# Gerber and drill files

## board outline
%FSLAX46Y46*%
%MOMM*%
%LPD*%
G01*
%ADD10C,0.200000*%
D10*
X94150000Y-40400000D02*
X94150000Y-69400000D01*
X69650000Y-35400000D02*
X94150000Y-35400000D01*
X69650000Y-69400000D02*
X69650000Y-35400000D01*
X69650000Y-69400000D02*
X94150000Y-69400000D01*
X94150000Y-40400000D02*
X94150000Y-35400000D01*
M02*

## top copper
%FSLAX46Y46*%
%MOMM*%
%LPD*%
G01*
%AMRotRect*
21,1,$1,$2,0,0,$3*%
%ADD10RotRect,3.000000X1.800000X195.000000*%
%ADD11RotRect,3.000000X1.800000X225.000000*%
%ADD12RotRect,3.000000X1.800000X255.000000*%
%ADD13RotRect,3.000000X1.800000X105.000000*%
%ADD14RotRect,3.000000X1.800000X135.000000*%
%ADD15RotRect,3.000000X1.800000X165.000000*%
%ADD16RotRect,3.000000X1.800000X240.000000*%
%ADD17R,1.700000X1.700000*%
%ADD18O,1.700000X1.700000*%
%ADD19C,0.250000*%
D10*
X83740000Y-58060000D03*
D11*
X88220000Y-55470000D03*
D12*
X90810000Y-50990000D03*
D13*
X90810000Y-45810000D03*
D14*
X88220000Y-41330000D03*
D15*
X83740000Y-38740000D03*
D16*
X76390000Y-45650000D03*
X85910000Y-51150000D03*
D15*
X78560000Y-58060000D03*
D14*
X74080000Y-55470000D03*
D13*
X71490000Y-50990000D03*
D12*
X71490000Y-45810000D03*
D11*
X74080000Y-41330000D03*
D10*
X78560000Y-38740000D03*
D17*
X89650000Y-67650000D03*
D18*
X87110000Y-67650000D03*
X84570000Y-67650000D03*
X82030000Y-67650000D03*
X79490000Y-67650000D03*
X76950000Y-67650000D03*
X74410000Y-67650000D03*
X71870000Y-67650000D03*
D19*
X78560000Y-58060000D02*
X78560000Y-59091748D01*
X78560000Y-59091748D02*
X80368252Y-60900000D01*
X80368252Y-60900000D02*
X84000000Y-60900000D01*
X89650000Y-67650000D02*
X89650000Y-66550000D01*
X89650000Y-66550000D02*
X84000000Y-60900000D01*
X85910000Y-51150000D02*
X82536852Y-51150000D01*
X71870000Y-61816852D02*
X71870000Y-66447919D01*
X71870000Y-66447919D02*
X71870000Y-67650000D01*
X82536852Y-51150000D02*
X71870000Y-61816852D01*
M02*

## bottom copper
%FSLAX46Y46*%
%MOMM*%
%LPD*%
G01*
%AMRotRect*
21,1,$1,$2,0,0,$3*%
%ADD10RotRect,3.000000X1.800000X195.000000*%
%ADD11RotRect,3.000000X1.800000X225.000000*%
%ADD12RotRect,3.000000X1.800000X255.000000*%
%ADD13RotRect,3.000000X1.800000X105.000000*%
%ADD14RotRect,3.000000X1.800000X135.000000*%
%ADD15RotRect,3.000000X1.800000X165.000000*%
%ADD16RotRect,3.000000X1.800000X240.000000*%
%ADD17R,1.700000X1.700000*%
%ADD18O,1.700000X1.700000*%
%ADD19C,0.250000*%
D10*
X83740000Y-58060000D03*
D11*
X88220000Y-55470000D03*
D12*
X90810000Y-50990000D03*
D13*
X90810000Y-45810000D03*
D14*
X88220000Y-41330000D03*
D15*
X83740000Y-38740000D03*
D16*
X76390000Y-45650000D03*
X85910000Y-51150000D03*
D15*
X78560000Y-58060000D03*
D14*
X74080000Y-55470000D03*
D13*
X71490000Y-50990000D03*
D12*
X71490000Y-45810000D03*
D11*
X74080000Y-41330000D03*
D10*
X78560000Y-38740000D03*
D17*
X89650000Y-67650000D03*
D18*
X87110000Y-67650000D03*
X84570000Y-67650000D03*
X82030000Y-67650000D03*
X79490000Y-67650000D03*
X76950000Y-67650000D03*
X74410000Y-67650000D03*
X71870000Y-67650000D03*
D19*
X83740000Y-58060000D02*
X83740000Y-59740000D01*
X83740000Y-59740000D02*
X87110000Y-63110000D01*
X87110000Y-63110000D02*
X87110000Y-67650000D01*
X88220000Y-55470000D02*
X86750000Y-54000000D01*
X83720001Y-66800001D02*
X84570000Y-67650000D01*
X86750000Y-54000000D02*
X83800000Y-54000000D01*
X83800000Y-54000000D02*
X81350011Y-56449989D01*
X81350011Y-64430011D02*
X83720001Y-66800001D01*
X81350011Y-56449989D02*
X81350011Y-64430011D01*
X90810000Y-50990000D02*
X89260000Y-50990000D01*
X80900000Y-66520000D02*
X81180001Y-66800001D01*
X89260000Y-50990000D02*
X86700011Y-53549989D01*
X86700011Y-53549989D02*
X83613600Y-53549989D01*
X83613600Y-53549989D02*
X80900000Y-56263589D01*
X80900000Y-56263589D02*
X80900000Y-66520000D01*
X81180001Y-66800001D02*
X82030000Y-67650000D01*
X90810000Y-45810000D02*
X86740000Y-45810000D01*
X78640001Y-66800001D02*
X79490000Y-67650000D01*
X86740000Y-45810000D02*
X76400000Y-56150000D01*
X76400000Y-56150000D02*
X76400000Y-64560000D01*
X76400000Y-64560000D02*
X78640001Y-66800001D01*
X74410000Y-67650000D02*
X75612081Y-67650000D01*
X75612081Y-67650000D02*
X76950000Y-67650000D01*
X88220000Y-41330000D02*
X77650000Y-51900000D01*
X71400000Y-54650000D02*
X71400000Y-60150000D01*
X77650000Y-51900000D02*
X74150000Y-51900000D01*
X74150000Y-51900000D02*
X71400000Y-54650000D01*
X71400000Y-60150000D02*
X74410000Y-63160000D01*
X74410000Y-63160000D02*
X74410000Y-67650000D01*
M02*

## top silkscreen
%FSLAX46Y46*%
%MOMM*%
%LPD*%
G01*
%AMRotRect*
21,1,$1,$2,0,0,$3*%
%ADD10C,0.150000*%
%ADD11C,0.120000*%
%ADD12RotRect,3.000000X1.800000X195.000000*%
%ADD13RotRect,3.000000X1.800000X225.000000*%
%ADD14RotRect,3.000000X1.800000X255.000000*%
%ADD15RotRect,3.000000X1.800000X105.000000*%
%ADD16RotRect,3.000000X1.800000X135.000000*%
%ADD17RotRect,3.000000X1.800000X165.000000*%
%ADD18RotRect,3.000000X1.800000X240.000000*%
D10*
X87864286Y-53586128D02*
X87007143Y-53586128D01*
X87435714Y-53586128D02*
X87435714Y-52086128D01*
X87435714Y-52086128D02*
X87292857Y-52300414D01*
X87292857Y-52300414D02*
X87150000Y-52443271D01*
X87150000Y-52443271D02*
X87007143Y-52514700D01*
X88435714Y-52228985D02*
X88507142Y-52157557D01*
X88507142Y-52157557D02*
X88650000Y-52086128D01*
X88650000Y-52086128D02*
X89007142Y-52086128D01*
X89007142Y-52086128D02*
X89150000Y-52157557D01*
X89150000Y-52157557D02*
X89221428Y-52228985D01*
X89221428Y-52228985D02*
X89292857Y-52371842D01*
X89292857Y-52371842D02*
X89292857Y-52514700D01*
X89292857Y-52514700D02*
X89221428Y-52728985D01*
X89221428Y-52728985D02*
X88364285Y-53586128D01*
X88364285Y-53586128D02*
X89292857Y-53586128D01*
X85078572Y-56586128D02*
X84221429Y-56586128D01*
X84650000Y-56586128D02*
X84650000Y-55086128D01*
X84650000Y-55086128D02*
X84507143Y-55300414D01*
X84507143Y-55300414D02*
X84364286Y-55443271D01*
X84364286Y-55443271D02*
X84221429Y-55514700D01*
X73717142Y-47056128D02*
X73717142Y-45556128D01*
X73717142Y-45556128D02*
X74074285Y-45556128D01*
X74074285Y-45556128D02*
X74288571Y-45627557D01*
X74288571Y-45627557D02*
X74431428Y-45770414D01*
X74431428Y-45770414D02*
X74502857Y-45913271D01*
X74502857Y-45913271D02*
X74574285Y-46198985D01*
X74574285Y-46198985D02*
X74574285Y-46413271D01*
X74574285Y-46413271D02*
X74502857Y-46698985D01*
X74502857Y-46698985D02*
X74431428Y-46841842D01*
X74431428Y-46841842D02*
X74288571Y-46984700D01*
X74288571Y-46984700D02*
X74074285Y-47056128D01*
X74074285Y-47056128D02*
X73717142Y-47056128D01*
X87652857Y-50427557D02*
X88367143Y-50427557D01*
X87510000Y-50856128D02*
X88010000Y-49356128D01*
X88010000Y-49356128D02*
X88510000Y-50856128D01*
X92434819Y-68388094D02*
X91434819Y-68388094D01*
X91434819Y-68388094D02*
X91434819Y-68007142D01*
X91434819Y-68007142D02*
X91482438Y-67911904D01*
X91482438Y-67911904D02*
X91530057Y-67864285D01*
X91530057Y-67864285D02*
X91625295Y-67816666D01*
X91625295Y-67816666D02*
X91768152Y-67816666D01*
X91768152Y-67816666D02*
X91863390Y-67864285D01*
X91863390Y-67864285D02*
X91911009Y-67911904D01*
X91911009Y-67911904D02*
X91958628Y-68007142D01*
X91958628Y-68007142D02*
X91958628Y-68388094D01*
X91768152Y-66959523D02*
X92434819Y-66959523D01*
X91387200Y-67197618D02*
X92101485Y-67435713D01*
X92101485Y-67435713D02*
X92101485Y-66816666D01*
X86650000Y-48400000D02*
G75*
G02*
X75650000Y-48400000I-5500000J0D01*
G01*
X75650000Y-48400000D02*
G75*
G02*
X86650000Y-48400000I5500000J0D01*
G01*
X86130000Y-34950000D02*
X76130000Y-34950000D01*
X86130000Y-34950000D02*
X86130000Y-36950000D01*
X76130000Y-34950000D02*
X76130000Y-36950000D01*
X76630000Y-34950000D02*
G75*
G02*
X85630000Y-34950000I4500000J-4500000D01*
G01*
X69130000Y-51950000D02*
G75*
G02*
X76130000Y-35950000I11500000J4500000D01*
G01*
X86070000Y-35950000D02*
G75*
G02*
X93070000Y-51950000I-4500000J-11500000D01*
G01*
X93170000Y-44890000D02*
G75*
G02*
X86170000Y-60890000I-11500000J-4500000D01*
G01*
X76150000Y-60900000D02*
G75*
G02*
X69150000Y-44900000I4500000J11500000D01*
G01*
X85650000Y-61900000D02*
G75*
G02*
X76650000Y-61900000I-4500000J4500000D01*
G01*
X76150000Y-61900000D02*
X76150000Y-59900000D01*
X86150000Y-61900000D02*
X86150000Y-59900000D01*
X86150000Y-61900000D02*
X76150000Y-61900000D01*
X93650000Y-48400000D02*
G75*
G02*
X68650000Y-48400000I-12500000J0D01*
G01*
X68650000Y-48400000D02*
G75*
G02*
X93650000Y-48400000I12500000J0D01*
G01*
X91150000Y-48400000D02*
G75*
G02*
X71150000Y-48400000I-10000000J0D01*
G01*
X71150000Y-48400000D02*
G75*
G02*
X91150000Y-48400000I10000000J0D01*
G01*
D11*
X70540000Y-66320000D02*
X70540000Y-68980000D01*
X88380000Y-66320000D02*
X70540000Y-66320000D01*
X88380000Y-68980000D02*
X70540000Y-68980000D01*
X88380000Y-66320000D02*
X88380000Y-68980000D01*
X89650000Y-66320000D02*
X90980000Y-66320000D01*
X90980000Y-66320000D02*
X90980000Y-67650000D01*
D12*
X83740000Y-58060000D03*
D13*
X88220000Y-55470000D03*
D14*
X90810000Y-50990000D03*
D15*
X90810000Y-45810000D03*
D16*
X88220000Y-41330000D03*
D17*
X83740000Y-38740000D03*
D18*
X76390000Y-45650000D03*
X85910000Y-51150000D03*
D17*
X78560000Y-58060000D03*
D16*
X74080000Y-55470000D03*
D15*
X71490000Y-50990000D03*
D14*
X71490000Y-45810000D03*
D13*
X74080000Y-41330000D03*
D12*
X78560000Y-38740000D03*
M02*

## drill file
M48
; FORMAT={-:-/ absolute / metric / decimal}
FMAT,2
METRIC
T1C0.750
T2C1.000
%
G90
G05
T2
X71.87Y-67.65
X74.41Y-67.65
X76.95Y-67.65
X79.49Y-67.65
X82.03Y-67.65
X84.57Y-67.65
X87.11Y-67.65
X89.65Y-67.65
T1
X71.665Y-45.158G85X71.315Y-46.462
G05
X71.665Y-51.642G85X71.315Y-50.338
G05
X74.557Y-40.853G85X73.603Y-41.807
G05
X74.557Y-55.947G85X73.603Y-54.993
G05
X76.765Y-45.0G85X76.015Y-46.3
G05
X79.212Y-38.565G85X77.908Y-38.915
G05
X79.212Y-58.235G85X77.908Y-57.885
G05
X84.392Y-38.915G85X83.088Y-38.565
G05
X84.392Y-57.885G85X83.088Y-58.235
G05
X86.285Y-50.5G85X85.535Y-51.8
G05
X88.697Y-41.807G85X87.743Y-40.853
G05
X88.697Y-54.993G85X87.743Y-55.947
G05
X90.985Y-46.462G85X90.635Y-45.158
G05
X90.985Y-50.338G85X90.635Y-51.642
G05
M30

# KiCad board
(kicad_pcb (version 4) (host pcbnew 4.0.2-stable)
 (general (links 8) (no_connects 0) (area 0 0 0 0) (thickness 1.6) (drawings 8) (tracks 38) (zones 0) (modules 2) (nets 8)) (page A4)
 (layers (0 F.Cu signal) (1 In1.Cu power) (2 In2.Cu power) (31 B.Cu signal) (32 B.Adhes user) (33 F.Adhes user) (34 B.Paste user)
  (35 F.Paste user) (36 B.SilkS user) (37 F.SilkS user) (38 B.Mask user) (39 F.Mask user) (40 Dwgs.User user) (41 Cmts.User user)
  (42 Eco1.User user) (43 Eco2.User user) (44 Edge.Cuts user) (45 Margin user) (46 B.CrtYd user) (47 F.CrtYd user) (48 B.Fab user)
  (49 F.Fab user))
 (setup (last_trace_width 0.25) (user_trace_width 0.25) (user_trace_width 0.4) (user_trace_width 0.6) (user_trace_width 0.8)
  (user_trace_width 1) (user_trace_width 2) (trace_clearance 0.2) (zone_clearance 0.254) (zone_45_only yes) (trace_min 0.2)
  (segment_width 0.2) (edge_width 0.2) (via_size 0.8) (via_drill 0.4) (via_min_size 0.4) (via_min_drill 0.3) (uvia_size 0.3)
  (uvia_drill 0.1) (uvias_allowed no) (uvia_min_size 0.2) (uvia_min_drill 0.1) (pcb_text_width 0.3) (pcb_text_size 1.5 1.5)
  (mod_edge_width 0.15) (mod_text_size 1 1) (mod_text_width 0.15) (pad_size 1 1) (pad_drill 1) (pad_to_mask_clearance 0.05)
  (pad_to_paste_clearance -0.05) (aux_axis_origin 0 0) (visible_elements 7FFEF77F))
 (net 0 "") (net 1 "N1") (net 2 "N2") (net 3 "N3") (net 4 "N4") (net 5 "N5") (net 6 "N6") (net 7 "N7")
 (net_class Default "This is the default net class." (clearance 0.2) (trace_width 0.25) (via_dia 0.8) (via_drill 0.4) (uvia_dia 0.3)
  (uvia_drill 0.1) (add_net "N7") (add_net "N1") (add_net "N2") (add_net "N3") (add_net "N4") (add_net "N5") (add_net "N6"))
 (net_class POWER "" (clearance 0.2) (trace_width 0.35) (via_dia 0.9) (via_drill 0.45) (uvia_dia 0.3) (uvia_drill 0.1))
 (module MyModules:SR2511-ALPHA (layer F.Cu) (at 81.15 48.4 180)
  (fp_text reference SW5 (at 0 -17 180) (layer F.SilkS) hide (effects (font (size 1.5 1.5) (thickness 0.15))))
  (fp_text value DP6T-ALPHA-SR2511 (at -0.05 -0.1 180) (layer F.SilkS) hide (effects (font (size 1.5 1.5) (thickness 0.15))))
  (fp_circle (center 0 0) (end 0 -5.5) (layer F.SilkS) (width 0.15))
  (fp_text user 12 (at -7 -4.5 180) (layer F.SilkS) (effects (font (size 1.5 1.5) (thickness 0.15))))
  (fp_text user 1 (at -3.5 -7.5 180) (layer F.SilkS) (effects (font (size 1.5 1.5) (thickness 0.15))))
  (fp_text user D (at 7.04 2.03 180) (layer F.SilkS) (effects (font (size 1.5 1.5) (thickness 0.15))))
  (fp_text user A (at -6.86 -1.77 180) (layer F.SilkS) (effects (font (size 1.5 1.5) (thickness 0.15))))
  (fp_line (start -4.98 13.45) (end 5.02 13.45) (layer F.SilkS) (width 0.15))
  (fp_line (start -4.98 13.45) (end -4.98 11.45) (layer F.SilkS) (width 0.15))
  (fp_line (start 5.02 13.45) (end 5.02 11.45) (layer F.SilkS) (width 0.15))
  (fp_arc (start 0.02 8.95) (end -4.48 13.45) (angle -90) (layer F.SilkS) (width 0.15))
  (fp_arc (start 0.52 0.95) (end 5.02 12.45) (angle -90) (layer F.SilkS) (width 0.15))
  (fp_arc (start -0.42 0.95) (end -4.92 12.45) (angle 90) (layer F.SilkS) (width 0.15))
  (fp_arc (start -0.52 -0.99) (end -5.02 -12.49) (angle -90) (layer F.SilkS) (width 0.15))
  (fp_arc (start 0.5 -1) (end 5 -12.5) (angle 90) (layer F.SilkS) (width 0.15))
  (fp_arc (start 0 -9) (end -4.5 -13.5) (angle 90) (layer F.SilkS) (width 0.15))
  (fp_line (start 5 -13.5) (end 5 -11.5) (layer F.SilkS) (width 0.15))
  (fp_line (start -5 -13.5) (end -5 -11.5) (layer F.SilkS) (width 0.15))
  (fp_line (start -5 -13.5) (end 5 -13.5) (layer F.SilkS) (width 0.15))
  (fp_circle (center 0 0) (end 12.5 0) (layer F.SilkS) (width 0.15))
  (fp_circle (center 0 0) (end 0 -10) (layer F.SilkS) (width 0.15))
  (pad 1 thru_hole rect (at -2.59 -9.66 195) (size 3 1.8) (drill oval 2.1 0.75) (layers *.Cu *.Mask F.SilkS) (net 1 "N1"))
  (pad 12 thru_hole rect (at -7.07 -7.07 225) (size 3 1.8) (drill oval 2.1 0.75) (layers *.Cu *.Mask F.SilkS) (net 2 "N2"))
  (pad 11 thru_hole rect (at -9.66 -2.59 255) (size 3 1.8) (drill oval 2.1 0.75) (layers *.Cu *.Mask F.SilkS) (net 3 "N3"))
  (pad 10 thru_hole rect (at -9.66 2.59 105) (size 3 1.8) (drill oval 2.1 0.75) (layers *.Cu *.Mask F.SilkS) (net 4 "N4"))
  (pad 9 thru_hole rect (at -7.07 7.07 135) (size 3 1.8) (drill oval 2.1 0.75) (layers *.Cu *.Mask F.SilkS) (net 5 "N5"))
  (pad 8 thru_hole rect (at -2.59 9.66 165) (size 3 1.8) (drill oval 2.1 0.75) (layers *.Cu *.Mask F.SilkS))
  (pad D thru_hole rect (at 4.76 2.75 240) (size 3 1.8) (drill oval 2.25 0.75) (layers *.Cu *.Mask F.SilkS))
  (pad A thru_hole rect (at -4.76 -2.75 240) (size 3 1.8) (drill oval 2.25 0.75) (layers *.Cu *.Mask F.SilkS) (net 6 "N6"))
  (pad 2 thru_hole rect (at 2.59 -9.66 165) (size 3 1.8) (drill oval 2.1 0.75) (layers *.Cu *.Mask F.SilkS) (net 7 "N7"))
  (pad 3 thru_hole rect (at 7.07 -7.07 135) (size 3 1.8) (drill oval 2.1 0.75) (layers *.Cu *.Mask F.SilkS))
  (pad 4 thru_hole rect (at 9.66 -2.59 105) (size 3 1.8) (drill oval 2.1 0.75) (layers *.Cu *.Mask F.SilkS))
  (pad 5 thru_hole rect (at 9.66 2.59 255) (size 3 1.8) (drill oval 2.1 0.75) (layers *.Cu *.Mask F.SilkS))
  (pad 6 thru_hole rect (at 7.07 7.07 225) (size 3 1.8) (drill oval 2.1 0.75) (layers *.Cu *.Mask F.SilkS))
  (pad 7 thru_hole rect (at 2.59 9.66 195) (size 3 1.8) (drill oval 2.1 0.75) (layers *.Cu *.Mask F.SilkS)))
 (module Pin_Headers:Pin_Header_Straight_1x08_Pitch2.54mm (layer F.Cu) (at 89.65 67.65 270)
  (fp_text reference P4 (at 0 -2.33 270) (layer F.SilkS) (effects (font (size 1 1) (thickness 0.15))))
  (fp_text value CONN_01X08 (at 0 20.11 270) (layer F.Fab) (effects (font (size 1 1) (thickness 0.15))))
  (fp_line (start -1.33 19.11) (end 1.33 19.11) (layer F.SilkS) (width 0.12))
  (fp_line (start -1.33 1.27) (end -1.33 19.11) (layer F.SilkS) (width 0.12))
  (fp_line (start 1.33 1.27) (end 1.33 19.11) (layer F.SilkS) (width 0.12))
  (fp_line (start -1.33 1.27) (end 1.33 1.27) (layer F.SilkS) (width 0.12))
  (fp_line (start -1.33 0) (end -1.33 -1.33) (layer F.SilkS) (width 0.12))
  (fp_line (start -1.33 -1.33) (end 0 -1.33) (layer F.SilkS) (width 0.12))
  (pad 1 thru_hole rect (at 0 0 270) (size 1.7 1.7) (drill 1) (layers *.Cu *.Mask) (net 7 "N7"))
  (pad 2 thru_hole oval (at 0 2.54 270) (size 1.7 1.7) (drill 1) (layers *.Cu *.Mask) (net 1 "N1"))
  (pad 3 thru_hole oval (at 0 5.08 270) (size 1.7 1.7) (drill 1) (layers *.Cu *.Mask) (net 2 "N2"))
  (pad 4 thru_hole oval (at 0 7.62 270) (size 1.7 1.7) (drill 1) (layers *.Cu *.Mask) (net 3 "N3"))
  (pad 5 thru_hole oval (at 0 10.16 270) (size 1.7 1.7) (drill 1) (layers *.Cu *.Mask) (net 4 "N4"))
  (pad 6 thru_hole oval (at 0 12.7 270) (size 1.7 1.7) (drill 1) (layers *.Cu *.Mask) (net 5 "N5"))
  (pad 7 thru_hole oval (at 0 15.24 270) (size 1.7 1.7) (drill 1) (layers *.Cu *.Mask) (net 5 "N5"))
  (pad 8 thru_hole oval (at 0 17.78 270) (size 1.7 1.7) (drill 1) (layers *.Cu *.Mask) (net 6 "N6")))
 (gr_line (start 94.15 40.4) (end 94.15 69.4) (layer Edge.Cuts) (width 0.2))
 (gr_line (start 69.65 35.4) (end 94.15 35.4) (layer Edge.Cuts) (width 0.2))
 (gr_line (start 69.65 69.4) (end 69.65 35.4) (layer Edge.Cuts) (width 0.2))
 (gr_line (start 69.65 69.4) (end 94.15 69.4) (layer Edge.Cuts) (width 0.2))
 (gr_line (start 94.15 40.4) (end 94.15 35.4) (layer Edge.Cuts) (width 0.2))
 (segment (start 78.56 58.06) (end 78.56 59.091748) (width 0.25) (layer F.Cu) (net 7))
 (segment (start 78.56 59.091748) (end 80.368252 60.9) (width 0.25) (layer F.Cu) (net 7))
 (segment (start 80.368252 60.9) (end 84 60.9) (width 0.25) (layer F.Cu) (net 7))
 (segment (start 89.65 67.65) (end 89.65 66.55) (width 0.25) (layer F.Cu) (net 7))
 (segment (start 89.65 66.55) (end 84 60.9) (width 0.25) (layer F.Cu) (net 7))
 (segment (start 83.74 58.06) (end 83.74 59.74) (width 0.25) (layer B.Cu) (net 1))
 (segment (start 83.74 59.74) (end 87.11 63.11) (width 0.25) (layer B.Cu) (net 1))
 (segment (start 87.11 63.11) (end 87.11 67.65) (width 0.25) (layer B.Cu) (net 1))
 (segment (start 88.22 55.47) (end 86.75 54) (width 0.25) (layer B.Cu) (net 2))
 (segment (start 83.720001 66.800001) (end 84.57 67.65) (width 0.25) (layer B.Cu) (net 2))
 (segment (start 86.75 54) (end 83.8 54) (width 0.25) (layer B.Cu) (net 2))
 (segment (start 83.8 54) (end 81.350011 56.449989) (width 0.25) (layer B.Cu) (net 2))
 (segment (start 81.350011 64.430011) (end 83.720001 66.800001) (width 0.25) (layer B.Cu) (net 2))
 (segment (start 81.350011 56.449989) (end 81.350011 64.430011) (width 0.25) (layer B.Cu) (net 2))
 (segment (start 90.81 50.99) (end 89.26 50.99) (width 0.25) (layer B.Cu) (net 3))
 (segment (start 80.9 66.52) (end 81.180001 66.800001) (width 0.25) (layer B.Cu) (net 3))
 (segment (start 89.26 50.99) (end 86.700011 53.549989) (width 0.25) (layer B.Cu) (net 3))
 (segment (start 86.700011 53.549989) (end 83.6136 53.549989) (width 0.25) (layer B.Cu) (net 3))
 (segment (start 83.6136 53.549989) (end 80.9 56.263589) (width 0.25) (layer B.Cu) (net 3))
 (segment (start 80.9 56.263589) (end 80.9 66.52) (width 0.25) (layer B.Cu) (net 3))
 (segment (start 81.180001 66.800001) (end 82.03 67.65) (width 0.25) (layer B.Cu) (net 3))
 (segment (start 90.81 45.81) (end 86.74 45.81) (width 0.25) (layer B.Cu) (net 4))
 (segment (start 78.640001 66.800001) (end 79.49 67.65) (width 0.25) (layer B.Cu) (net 4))
 (segment (start 86.74 45.81) (end 76.4 56.15) (width 0.25) (layer B.Cu) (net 4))
 (segment (start 76.4 56.15) (end 76.4 64.56) (width 0.25) (layer B.Cu) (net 4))
 (segment (start 76.4 64.56) (end 78.640001 66.800001) (width 0.25) (layer B.Cu) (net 4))
 (segment (start 74.41 67.65) (end 75.612081 67.65) (width 0.25) (layer B.Cu) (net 5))
 (segment (start 75.612081 67.65) (end 76.95 67.65) (width 0.25) (layer B.Cu) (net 5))
 (segment (start 88.22 41.33) (end 77.65 51.9) (width 0.25) (layer B.Cu) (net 5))
 (segment (start 71.4 54.65) (end 71.4 60.15) (width 0.25) (layer B.Cu) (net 5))
 (segment (start 77.65 51.9) (end 74.15 51.9) (width 0.25) (layer B.Cu) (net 5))
 (segment (start 74.15 51.9) (end 71.4 54.65) (width 0.25) (layer B.Cu) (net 5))
 (segment (start 71.4 60.15) (end 74.41 63.16) (width 0.25) (layer B.Cu) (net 5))
 (segment (start 74.41 63.16) (end 74.41 67.65) (width 0.25) (layer B.Cu) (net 5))
 (segment (start 85.91 51.15) (end 82.536852 51.15) (width 0.25) (layer F.Cu) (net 6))
 (segment (start 71.87 61.816852) (end 71.87 66.447919) (width 0.25) (layer F.Cu) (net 6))
 (segment (start 71.87 66.447919) (end 71.87 67.65) (width 0.25) (layer F.Cu) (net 6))
 (segment (start 82.536852 51.15) (end 71.87 61.816852) (width 0.25) (layer F.Cu) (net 6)))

